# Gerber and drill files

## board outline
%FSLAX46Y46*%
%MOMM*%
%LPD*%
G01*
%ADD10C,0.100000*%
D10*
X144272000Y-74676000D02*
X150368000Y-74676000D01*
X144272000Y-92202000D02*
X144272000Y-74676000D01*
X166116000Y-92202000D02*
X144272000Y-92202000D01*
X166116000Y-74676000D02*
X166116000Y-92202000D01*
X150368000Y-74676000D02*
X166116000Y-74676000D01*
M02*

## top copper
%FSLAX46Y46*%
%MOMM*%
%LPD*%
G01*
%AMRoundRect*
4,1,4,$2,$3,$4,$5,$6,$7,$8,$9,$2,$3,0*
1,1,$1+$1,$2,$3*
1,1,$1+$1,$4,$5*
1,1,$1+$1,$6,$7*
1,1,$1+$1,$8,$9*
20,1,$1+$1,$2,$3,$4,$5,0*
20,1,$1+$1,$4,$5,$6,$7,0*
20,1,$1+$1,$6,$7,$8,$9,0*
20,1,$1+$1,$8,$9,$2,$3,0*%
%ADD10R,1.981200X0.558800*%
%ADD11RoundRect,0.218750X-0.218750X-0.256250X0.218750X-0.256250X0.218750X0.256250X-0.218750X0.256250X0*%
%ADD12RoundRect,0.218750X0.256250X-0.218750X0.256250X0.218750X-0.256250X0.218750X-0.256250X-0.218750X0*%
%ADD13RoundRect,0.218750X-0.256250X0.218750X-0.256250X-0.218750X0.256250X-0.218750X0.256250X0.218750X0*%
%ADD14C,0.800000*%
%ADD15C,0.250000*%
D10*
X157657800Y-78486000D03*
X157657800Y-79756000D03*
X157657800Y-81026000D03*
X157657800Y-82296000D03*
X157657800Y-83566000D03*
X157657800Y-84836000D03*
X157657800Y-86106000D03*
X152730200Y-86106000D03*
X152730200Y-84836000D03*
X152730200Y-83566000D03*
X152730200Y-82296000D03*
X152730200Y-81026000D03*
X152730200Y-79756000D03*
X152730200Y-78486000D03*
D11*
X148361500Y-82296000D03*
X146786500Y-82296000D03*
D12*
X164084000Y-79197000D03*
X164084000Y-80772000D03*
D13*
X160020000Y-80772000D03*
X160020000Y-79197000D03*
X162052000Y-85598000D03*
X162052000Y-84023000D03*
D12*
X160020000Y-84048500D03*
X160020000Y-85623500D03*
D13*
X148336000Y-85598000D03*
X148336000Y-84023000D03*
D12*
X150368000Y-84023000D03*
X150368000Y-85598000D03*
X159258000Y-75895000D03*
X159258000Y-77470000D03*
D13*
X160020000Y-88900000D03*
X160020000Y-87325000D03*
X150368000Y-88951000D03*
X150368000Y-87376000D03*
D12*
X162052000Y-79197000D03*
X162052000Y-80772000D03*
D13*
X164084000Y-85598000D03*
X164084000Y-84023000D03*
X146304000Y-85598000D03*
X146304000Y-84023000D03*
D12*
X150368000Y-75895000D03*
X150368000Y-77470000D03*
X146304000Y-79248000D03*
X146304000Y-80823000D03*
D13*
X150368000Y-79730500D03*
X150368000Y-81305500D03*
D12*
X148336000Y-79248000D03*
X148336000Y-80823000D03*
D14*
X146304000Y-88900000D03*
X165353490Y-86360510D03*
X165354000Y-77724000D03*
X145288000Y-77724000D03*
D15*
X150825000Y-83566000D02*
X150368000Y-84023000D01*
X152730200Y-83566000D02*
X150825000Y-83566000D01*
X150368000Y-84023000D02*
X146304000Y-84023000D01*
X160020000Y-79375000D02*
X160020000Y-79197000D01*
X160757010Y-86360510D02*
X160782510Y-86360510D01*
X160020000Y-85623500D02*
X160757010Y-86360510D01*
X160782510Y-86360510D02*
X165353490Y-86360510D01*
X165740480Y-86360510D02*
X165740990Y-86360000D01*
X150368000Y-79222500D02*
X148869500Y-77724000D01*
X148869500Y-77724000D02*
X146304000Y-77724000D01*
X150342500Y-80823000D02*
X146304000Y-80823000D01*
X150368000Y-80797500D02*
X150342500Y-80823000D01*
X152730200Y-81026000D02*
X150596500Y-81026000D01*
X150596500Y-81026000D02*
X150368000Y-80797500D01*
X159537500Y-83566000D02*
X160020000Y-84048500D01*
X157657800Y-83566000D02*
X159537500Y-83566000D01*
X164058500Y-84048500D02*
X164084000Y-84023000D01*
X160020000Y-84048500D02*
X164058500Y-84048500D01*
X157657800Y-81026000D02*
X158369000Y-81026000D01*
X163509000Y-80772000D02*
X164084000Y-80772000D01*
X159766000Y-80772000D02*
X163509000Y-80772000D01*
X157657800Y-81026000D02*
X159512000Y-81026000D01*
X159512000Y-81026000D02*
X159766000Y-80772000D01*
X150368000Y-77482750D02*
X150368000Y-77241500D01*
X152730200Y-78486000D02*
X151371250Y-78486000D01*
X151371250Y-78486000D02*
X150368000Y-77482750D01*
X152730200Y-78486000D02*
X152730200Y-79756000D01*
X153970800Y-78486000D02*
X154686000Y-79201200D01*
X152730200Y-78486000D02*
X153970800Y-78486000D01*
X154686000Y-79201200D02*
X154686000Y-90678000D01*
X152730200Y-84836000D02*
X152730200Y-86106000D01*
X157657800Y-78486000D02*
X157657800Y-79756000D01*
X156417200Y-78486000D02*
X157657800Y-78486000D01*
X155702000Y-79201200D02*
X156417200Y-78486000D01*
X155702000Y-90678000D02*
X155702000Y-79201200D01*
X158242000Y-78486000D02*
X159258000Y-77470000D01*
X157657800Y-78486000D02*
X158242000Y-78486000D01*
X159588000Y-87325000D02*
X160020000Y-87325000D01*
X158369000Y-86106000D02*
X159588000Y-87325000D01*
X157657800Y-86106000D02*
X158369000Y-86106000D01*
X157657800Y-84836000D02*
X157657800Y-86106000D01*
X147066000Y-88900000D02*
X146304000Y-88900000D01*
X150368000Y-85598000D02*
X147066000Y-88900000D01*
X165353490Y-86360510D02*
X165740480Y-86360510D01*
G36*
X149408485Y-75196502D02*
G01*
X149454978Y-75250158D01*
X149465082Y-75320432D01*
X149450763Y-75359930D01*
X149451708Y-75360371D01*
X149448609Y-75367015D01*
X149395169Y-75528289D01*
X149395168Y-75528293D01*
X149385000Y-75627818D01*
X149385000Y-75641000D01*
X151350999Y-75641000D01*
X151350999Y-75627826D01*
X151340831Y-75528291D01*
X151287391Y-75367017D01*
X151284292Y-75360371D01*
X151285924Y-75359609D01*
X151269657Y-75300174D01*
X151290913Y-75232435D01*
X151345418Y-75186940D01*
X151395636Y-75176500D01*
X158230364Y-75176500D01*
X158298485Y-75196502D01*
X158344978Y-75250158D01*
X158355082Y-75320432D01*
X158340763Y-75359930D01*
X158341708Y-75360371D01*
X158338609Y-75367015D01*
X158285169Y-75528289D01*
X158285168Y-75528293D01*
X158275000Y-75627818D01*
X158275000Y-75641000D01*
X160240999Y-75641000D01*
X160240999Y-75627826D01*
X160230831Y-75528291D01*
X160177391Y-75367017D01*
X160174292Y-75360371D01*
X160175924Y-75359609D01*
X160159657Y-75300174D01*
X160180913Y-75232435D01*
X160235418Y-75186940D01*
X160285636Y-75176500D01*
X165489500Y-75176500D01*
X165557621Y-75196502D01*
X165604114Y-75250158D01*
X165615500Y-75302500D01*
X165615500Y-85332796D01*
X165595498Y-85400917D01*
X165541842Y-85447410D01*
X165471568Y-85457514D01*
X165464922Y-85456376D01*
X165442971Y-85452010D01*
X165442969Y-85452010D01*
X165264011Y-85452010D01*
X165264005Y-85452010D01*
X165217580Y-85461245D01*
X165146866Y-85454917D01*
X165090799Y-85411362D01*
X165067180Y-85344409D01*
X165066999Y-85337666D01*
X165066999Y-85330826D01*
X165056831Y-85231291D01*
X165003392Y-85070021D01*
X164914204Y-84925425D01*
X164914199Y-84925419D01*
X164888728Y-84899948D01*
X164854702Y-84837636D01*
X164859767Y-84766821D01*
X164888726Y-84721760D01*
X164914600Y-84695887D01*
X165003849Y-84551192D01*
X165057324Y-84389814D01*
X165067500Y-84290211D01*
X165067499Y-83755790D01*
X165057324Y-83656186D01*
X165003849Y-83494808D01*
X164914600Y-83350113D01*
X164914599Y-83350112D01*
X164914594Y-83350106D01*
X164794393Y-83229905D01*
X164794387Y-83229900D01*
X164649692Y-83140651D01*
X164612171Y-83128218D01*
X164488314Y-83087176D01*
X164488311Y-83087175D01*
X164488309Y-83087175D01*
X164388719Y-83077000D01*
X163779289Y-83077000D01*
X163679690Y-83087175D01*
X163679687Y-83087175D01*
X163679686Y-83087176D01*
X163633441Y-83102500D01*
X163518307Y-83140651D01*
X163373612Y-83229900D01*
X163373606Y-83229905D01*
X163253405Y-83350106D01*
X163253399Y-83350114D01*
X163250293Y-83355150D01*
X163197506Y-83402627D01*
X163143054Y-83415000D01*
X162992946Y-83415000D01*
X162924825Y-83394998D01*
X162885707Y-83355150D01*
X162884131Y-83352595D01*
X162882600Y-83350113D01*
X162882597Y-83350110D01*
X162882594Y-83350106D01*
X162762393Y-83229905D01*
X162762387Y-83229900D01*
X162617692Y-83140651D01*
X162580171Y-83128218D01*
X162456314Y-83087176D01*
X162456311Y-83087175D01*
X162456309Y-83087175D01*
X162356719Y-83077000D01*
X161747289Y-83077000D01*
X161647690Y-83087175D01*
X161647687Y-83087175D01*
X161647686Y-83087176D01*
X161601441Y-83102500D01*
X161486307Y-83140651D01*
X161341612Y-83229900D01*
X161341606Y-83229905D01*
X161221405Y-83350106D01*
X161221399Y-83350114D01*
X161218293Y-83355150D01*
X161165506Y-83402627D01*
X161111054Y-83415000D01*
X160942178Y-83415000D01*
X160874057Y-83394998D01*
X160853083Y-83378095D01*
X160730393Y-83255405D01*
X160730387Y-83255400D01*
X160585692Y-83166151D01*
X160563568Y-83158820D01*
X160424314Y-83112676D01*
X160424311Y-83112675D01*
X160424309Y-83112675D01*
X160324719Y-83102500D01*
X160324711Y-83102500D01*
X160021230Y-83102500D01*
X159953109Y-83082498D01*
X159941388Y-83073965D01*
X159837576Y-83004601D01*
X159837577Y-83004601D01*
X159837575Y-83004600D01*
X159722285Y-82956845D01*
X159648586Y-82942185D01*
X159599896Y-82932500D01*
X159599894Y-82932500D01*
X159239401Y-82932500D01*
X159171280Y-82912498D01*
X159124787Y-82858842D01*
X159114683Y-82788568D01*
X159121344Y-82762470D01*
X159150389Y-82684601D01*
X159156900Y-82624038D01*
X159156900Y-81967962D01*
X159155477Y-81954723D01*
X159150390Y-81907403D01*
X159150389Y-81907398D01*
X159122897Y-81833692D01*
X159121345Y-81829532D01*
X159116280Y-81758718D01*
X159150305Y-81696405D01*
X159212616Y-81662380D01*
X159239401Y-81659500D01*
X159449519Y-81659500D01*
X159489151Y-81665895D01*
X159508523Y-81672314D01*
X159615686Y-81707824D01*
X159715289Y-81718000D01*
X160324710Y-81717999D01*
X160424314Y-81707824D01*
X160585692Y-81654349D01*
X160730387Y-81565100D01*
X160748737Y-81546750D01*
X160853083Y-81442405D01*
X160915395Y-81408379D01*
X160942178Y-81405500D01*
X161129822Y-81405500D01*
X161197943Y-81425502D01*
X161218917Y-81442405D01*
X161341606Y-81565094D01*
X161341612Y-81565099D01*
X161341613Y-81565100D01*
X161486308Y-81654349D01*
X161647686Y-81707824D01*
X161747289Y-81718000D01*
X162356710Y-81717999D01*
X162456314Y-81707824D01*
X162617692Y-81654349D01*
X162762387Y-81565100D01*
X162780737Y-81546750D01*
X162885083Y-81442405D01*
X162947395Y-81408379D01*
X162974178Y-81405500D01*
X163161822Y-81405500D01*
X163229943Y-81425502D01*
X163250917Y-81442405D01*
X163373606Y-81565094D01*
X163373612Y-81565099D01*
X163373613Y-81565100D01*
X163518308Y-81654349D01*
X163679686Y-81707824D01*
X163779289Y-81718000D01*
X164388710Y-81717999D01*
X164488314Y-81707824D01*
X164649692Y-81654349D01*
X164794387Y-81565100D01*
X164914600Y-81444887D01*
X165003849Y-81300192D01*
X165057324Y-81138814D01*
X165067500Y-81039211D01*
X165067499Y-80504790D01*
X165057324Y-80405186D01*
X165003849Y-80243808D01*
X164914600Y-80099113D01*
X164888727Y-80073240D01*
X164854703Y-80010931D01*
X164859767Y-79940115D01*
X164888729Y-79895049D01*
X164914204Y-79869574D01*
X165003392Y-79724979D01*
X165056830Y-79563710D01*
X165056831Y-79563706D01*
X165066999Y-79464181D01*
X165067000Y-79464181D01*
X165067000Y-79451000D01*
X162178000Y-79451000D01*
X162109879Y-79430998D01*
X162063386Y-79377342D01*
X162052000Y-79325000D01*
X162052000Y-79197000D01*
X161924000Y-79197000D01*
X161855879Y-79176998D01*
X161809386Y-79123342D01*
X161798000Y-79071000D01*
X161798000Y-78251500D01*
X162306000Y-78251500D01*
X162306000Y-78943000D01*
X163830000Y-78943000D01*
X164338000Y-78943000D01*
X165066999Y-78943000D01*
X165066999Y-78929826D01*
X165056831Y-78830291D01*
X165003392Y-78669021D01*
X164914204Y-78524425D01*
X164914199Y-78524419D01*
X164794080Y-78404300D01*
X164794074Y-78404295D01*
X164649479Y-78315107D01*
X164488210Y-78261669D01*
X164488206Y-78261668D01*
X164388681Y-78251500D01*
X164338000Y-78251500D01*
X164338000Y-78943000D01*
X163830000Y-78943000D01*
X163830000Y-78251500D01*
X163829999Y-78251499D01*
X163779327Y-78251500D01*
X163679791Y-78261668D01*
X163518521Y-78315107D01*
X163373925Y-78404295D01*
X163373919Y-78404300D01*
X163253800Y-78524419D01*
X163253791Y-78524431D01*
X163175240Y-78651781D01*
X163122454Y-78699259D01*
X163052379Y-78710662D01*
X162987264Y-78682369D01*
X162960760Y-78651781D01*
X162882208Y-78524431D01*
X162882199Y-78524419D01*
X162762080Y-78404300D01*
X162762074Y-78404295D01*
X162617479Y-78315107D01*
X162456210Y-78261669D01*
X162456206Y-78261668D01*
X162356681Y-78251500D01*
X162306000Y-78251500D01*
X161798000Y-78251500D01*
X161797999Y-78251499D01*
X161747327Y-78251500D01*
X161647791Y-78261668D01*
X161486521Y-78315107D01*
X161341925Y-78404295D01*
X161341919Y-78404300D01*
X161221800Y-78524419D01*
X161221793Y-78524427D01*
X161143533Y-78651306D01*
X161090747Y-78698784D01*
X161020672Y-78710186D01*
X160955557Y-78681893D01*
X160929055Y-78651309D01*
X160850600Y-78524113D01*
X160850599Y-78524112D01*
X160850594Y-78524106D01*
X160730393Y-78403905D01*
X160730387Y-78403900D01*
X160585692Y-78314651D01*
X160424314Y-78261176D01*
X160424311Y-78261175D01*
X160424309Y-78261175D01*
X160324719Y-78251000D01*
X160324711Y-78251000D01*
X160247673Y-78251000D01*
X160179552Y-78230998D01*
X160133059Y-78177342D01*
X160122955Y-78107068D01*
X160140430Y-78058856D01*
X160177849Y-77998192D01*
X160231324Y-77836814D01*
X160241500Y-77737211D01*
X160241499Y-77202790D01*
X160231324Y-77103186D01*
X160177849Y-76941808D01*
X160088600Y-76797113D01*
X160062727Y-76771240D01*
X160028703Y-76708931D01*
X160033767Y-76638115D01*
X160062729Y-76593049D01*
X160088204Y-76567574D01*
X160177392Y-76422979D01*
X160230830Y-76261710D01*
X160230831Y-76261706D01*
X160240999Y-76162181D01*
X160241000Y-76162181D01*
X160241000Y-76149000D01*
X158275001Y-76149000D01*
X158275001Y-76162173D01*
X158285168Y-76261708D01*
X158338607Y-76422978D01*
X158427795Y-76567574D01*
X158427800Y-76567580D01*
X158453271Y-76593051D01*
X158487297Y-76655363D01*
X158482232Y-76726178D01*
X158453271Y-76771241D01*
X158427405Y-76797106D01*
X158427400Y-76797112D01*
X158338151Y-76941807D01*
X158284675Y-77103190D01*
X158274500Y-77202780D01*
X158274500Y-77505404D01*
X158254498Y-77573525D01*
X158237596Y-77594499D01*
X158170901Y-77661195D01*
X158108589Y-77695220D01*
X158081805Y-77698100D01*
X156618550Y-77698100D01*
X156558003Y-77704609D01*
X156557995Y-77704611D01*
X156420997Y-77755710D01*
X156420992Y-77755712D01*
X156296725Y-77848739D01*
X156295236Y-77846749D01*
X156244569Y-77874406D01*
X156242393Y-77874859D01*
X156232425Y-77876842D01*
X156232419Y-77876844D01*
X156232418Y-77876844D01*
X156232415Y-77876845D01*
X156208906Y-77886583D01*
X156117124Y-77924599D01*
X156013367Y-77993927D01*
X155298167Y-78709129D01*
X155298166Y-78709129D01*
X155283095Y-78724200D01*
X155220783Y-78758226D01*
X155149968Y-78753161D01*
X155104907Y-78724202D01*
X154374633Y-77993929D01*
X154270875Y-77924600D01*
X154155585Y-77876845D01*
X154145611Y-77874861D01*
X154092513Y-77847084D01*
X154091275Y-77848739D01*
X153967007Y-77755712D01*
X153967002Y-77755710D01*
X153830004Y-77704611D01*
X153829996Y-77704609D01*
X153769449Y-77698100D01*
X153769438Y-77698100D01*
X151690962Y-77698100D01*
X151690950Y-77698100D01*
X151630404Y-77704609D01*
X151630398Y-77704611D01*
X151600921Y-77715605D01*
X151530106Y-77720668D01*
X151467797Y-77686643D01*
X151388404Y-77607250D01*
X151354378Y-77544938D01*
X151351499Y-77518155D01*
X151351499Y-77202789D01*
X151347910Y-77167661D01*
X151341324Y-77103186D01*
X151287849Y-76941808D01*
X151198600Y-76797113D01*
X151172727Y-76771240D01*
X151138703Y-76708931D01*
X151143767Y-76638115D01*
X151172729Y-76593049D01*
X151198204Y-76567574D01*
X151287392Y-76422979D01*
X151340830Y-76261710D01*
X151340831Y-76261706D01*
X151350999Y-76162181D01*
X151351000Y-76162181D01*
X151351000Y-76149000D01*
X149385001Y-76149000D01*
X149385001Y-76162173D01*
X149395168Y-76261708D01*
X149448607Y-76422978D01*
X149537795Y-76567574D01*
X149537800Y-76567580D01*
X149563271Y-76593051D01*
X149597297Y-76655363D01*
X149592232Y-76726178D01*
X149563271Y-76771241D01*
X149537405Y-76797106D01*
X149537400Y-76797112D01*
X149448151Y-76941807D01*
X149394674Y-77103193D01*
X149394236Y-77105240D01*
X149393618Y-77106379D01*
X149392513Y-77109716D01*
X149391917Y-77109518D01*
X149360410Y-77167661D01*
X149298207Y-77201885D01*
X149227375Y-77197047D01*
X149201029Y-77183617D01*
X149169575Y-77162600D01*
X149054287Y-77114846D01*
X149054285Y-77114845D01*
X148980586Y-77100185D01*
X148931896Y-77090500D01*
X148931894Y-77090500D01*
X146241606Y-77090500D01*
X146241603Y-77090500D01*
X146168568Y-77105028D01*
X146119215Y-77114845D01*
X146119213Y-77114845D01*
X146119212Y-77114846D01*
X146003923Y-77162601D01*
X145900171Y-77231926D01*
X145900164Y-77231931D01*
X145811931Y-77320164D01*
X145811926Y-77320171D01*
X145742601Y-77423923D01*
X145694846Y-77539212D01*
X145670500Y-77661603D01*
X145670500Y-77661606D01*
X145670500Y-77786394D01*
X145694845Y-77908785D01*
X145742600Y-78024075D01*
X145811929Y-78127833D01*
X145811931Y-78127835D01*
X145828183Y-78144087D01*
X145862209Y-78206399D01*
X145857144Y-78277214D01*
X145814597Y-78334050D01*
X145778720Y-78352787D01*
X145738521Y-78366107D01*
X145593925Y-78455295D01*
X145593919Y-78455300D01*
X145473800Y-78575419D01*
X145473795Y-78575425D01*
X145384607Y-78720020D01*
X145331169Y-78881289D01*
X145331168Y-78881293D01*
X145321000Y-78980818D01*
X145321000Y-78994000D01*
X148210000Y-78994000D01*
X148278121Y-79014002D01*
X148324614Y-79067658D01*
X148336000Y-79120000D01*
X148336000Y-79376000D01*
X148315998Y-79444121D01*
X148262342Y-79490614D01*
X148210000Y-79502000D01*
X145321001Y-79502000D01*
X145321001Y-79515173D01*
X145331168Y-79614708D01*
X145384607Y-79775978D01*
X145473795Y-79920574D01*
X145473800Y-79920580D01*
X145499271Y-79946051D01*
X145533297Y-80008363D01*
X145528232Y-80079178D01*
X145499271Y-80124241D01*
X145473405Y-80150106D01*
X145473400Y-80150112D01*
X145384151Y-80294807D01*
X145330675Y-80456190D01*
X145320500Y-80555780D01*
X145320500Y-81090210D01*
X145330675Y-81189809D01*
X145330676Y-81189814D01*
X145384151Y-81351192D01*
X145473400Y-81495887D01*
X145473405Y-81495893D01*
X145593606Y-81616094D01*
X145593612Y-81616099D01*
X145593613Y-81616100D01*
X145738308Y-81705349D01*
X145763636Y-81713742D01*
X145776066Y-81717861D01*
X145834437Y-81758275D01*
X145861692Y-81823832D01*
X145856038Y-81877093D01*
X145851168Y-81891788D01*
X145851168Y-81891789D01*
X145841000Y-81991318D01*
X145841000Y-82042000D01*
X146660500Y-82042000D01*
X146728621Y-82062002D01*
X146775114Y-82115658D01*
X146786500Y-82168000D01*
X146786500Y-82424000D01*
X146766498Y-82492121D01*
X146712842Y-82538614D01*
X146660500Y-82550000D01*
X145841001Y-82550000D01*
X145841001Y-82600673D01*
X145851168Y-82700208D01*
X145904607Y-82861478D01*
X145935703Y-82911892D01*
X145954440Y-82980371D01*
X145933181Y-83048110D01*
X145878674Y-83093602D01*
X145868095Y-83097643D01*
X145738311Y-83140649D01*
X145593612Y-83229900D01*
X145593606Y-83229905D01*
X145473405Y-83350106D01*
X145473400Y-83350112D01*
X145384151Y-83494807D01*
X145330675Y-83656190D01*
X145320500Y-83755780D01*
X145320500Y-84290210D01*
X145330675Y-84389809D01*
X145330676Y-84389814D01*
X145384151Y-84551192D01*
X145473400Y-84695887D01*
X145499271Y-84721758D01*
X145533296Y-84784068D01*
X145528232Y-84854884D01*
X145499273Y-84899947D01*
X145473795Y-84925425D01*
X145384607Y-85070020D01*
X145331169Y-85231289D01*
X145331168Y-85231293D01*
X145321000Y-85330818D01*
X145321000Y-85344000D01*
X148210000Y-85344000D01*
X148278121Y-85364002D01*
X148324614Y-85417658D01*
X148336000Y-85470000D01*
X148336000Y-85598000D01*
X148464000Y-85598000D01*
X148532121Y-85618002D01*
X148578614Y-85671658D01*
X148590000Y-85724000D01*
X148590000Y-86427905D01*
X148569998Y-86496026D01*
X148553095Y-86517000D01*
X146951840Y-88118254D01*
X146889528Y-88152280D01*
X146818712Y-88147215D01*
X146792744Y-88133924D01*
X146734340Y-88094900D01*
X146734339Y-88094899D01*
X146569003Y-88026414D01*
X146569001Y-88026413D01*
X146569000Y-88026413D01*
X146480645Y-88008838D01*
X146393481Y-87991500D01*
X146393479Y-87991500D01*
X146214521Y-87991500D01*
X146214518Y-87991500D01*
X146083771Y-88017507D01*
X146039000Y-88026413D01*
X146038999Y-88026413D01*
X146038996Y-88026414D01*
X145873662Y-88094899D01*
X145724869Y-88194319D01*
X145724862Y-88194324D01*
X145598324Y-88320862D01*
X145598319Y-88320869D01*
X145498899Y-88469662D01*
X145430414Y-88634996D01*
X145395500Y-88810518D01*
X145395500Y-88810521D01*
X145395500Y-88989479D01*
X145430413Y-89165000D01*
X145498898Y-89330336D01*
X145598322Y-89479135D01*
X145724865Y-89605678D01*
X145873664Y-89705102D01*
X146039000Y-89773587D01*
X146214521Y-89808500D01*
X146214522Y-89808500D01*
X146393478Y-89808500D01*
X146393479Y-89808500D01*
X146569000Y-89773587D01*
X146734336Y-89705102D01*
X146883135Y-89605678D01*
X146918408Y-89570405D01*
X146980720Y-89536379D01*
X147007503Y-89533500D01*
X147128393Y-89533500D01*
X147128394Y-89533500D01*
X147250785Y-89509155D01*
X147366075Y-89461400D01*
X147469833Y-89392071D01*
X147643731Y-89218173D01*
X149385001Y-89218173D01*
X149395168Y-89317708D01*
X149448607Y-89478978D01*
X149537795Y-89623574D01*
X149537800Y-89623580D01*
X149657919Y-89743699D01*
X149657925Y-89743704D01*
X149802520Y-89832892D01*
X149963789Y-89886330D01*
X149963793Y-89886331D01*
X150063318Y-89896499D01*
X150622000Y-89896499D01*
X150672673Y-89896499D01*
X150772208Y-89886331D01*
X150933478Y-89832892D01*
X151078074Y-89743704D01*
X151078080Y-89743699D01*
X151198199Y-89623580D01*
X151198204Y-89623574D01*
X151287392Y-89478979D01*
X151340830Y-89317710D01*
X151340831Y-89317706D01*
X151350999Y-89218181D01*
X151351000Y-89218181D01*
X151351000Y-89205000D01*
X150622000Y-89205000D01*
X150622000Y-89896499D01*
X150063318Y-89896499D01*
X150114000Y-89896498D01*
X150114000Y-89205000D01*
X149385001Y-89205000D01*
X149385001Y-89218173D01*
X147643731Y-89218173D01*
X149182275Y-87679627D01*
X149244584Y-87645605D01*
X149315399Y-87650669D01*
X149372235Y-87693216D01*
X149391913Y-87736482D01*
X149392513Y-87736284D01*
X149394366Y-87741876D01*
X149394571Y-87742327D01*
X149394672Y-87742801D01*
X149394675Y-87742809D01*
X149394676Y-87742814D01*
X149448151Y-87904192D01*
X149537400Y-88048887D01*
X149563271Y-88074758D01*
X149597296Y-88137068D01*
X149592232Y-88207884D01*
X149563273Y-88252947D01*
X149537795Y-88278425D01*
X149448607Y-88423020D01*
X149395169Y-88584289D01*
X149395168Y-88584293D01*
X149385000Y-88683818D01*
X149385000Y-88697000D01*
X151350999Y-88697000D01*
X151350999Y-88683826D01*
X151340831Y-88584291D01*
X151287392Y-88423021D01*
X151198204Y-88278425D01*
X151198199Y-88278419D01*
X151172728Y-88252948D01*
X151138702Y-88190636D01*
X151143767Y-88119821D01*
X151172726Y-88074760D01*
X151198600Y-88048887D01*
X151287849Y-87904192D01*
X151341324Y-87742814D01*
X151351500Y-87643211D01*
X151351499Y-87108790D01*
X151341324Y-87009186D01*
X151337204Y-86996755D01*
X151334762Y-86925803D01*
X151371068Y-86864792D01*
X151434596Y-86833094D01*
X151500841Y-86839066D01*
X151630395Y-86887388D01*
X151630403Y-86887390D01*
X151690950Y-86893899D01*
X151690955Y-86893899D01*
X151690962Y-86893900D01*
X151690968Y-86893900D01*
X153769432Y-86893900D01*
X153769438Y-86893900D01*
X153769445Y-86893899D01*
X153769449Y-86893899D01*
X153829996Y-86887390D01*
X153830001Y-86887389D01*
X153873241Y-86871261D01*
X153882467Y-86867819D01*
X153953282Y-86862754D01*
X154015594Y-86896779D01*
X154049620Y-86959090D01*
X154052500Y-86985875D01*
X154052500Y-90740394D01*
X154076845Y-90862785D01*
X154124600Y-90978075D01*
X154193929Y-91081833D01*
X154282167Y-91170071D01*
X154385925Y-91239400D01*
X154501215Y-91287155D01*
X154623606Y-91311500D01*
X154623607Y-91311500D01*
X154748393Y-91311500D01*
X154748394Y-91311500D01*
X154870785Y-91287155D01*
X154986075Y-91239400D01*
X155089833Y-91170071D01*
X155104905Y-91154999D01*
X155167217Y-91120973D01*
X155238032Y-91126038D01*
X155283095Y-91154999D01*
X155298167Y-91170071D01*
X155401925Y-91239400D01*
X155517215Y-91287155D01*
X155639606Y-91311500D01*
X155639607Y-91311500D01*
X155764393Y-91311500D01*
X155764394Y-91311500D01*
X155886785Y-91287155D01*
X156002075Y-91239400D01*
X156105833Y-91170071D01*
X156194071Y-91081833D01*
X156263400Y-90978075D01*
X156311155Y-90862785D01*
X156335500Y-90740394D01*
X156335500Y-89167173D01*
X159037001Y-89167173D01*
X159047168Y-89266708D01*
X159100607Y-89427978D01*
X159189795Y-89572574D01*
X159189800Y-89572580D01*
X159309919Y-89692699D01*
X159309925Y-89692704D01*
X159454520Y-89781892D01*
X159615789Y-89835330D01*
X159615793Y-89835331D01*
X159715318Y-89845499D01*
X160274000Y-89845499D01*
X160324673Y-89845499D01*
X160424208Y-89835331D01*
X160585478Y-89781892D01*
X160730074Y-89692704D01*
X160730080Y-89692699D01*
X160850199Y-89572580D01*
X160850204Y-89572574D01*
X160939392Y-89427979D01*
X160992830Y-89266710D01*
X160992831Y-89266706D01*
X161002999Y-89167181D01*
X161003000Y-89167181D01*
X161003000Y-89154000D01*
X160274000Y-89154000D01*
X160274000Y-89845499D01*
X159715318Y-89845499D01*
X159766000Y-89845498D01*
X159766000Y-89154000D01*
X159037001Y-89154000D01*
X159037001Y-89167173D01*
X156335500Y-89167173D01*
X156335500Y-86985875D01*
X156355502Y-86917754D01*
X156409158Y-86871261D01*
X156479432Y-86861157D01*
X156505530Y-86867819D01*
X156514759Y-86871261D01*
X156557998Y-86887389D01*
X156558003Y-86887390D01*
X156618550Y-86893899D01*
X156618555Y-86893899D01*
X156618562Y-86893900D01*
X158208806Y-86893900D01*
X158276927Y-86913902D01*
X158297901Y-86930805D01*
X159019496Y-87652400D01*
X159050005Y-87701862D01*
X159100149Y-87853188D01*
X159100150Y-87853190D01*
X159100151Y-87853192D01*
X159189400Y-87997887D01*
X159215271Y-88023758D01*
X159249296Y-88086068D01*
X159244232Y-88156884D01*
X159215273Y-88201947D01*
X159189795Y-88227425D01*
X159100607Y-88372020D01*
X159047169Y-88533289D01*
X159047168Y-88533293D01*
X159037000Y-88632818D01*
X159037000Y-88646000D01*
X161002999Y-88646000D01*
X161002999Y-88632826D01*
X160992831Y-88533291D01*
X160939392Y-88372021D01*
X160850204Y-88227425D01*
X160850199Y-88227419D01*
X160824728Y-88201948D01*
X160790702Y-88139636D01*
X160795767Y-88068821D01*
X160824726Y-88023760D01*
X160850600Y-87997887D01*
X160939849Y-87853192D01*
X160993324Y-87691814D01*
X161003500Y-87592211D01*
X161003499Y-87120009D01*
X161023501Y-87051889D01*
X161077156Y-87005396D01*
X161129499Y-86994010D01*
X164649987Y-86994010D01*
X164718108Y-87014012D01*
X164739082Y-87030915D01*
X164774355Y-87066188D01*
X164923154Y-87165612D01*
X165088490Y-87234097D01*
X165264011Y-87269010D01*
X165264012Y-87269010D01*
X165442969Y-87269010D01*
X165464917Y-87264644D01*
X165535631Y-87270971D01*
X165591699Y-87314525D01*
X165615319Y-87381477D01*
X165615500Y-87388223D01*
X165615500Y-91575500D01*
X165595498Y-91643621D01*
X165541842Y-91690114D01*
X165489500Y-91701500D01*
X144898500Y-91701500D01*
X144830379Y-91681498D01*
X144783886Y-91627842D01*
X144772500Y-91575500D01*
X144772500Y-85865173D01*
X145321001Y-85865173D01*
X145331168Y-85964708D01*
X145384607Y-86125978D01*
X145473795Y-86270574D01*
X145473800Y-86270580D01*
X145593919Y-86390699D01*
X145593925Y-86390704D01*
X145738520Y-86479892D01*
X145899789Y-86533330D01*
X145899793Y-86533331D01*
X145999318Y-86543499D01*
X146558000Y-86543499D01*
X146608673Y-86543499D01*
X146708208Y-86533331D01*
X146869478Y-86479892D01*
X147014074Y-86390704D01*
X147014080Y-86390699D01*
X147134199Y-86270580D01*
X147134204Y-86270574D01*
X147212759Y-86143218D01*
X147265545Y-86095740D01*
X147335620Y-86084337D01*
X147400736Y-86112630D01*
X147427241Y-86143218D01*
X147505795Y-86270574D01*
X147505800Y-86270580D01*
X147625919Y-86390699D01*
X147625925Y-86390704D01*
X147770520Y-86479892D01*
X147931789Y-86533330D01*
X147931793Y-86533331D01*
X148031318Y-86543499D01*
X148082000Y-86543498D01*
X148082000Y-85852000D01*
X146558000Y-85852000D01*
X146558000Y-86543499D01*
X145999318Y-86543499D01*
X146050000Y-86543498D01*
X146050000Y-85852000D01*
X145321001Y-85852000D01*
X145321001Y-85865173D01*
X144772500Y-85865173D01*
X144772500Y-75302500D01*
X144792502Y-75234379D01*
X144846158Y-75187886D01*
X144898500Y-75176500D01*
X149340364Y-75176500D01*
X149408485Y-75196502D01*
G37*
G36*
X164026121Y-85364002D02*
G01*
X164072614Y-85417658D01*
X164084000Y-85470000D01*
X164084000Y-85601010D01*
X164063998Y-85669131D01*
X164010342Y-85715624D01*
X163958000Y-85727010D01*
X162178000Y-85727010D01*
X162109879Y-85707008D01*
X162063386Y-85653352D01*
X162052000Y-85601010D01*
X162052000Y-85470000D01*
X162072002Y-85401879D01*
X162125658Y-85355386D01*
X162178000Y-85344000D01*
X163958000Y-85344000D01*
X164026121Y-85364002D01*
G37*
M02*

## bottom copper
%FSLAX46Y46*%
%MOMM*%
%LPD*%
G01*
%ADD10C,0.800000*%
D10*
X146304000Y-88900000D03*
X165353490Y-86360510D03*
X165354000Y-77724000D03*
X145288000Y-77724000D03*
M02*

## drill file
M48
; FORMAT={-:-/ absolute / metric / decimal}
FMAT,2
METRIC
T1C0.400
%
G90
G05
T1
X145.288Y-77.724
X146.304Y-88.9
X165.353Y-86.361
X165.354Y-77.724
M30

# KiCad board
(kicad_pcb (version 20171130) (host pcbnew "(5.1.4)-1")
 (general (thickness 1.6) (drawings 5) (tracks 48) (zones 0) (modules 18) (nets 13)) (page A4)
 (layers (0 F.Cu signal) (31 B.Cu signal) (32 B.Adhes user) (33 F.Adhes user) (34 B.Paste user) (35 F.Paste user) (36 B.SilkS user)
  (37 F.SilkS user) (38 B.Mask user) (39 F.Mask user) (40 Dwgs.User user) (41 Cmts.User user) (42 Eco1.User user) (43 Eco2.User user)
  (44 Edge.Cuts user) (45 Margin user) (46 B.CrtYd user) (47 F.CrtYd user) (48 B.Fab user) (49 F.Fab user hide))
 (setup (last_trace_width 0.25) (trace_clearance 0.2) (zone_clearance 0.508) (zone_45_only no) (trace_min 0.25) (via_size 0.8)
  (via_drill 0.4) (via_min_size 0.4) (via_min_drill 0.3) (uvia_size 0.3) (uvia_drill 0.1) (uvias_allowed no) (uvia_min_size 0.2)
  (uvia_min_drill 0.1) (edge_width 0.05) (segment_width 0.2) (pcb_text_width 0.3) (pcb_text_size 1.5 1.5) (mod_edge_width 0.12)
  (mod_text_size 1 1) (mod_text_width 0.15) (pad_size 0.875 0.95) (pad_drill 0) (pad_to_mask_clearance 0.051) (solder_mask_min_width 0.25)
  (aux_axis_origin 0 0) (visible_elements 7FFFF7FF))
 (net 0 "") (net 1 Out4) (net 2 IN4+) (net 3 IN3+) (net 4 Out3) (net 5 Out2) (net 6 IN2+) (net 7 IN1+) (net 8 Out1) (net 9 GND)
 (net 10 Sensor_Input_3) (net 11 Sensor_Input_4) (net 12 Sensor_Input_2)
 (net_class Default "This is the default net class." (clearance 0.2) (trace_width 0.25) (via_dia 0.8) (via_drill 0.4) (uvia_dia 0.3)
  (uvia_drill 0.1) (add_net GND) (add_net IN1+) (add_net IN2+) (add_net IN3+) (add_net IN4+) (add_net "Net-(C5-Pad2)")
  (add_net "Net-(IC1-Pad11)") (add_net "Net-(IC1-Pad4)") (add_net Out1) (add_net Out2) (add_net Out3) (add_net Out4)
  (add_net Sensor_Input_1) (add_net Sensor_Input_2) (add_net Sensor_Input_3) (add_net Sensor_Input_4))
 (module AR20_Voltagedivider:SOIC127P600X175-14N (layer F.Cu) (at 155.194 82.296)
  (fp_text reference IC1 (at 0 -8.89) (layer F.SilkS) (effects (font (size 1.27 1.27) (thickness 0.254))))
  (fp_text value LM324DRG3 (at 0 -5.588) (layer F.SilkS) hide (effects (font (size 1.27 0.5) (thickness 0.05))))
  (pad 14 smd rect (at 2.4638 -3.81 90) (size 0.5588 1.9812) (layers F.Cu F.Paste F.Mask) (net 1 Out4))
  (pad 13 smd rect (at 2.4638 -2.54 90) (size 0.5588 1.9812) (layers F.Cu F.Paste F.Mask) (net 1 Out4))
  (pad 12 smd rect (at 2.4638 -1.27 90) (size 0.5588 1.9812) (layers F.Cu F.Paste F.Mask) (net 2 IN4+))
  (pad 11 smd rect (at 2.4638 0 90) (size 0.5588 1.9812) (layers F.Cu F.Paste F.Mask))
  (pad 10 smd rect (at 2.4638 1.27 90) (size 0.5588 1.9812) (layers F.Cu F.Paste F.Mask) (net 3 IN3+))
  (pad 9 smd rect (at 2.4638 2.54 90) (size 0.5588 1.9812) (layers F.Cu F.Paste F.Mask) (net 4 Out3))
  (pad 8 smd rect (at 2.4638 3.81 90) (size 0.5588 1.9812) (layers F.Cu F.Paste F.Mask) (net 4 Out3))
  (pad 7 smd rect (at -2.4638 3.81 90) (size 0.5588 1.9812) (layers F.Cu F.Paste F.Mask) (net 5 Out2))
  (pad 6 smd rect (at -2.4638 2.54 90) (size 0.5588 1.9812) (layers F.Cu F.Paste F.Mask) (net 5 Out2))
  (pad 5 smd rect (at -2.4638 1.27 90) (size 0.5588 1.9812) (layers F.Cu F.Paste F.Mask) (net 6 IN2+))
  (pad 4 smd rect (at -2.4638 0 90) (size 0.5588 1.9812) (layers F.Cu F.Paste F.Mask))
  (pad 3 smd rect (at -2.4638 -1.27 90) (size 0.5588 1.9812) (layers F.Cu F.Paste F.Mask) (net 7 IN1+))
  (pad 2 smd rect (at -2.4638 -2.54 90) (size 0.5588 1.9812) (layers F.Cu F.Paste F.Mask) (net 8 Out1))
  (pad 1 smd rect (at -2.4638 -3.81 90) (size 0.5588 1.9812) (layers F.Cu F.Paste F.Mask) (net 8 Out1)))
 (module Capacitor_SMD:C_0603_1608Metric (layer F.Cu) (at 147.574 82.296)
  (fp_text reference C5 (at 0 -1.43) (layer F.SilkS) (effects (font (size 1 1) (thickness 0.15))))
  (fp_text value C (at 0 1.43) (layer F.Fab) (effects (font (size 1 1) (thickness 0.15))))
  (pad 2 smd roundrect (at 0.7875 0) (size 0.875 0.95) (layers F.Cu F.Paste F.Mask) (roundrect_rratio 0.25))
  (pad 1 smd roundrect (at -0.7875 0) (size 0.875 0.95) (layers F.Cu F.Paste F.Mask) (roundrect_rratio 0.25) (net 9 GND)))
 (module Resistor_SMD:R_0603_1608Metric (layer F.Cu) (at 164.084 79.9845 90)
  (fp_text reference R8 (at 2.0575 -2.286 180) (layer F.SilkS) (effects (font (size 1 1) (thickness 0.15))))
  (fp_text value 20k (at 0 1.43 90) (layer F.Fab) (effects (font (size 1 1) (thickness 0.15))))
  (pad 2 smd roundrect (at 0.7875 0 90) (size 0.875 0.95) (layers F.Cu F.Paste F.Mask) (roundrect_rratio 0.25) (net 9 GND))
  (pad 1 smd roundrect (at -0.7875 0 90) (size 0.875 0.95) (layers F.Cu F.Paste F.Mask) (roundrect_rratio 0.25) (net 2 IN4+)))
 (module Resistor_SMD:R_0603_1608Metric (layer F.Cu) (at 160.02 79.9845 270)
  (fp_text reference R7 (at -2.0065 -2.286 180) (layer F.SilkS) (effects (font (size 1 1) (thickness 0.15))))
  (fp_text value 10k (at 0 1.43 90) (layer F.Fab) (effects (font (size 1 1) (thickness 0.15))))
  (pad 2 smd roundrect (at 0.7875 0 270) (size 0.875 0.95) (layers F.Cu F.Paste F.Mask) (roundrect_rratio 0.25) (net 2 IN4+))
  (pad 1 smd roundrect (at -0.7875 0 270) (size 0.875 0.95) (layers F.Cu F.Paste F.Mask) (roundrect_rratio 0.25)))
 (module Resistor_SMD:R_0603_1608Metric (layer F.Cu) (at 162.052 84.8105 270)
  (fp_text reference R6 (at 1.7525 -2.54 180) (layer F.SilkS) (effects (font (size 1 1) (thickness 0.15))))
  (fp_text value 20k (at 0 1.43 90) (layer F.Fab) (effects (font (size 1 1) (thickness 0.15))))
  (pad 2 smd roundrect (at 0.7875 0 270) (size 0.875 0.95) (layers F.Cu F.Paste F.Mask) (roundrect_rratio 0.25) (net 9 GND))
  (pad 1 smd roundrect (at -0.7875 0 270) (size 0.875 0.95) (layers F.Cu F.Paste F.Mask) (roundrect_rratio 0.25) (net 3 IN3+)))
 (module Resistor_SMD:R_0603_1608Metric (layer F.Cu) (at 160.02 84.836 90)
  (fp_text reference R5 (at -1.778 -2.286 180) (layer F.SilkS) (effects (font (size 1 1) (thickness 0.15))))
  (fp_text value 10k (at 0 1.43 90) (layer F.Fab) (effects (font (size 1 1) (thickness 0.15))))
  (pad 2 smd roundrect (at 0.7875 0 90) (size 0.875 0.95) (layers F.Cu F.Paste F.Mask) (roundrect_rratio 0.25) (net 3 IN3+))
  (pad 1 smd roundrect (at -0.7875 0 90) (size 0.875 0.95) (layers F.Cu F.Paste F.Mask) (roundrect_rratio 0.25)))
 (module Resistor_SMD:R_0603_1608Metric (layer F.Cu) (at 148.336 84.8105 270)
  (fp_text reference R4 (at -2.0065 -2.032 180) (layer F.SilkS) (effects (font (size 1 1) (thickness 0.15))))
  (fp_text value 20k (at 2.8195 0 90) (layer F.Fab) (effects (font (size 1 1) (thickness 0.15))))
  (pad 2 smd roundrect (at 0.7875 0 270) (size 0.875 0.95) (layers F.Cu F.Paste F.Mask) (roundrect_rratio 0.25) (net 9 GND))
  (pad 1 smd roundrect (at -0.7875 0 270) (size 0.875 0.95) (layers F.Cu F.Paste F.Mask) (roundrect_rratio 0.25) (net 6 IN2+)))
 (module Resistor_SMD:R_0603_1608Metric (layer F.Cu) (at 150.368 84.8105 90)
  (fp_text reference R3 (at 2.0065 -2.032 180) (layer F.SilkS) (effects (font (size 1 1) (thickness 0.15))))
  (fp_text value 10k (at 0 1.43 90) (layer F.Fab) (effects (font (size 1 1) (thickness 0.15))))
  (pad 2 smd roundrect (at 0.7875 0 90) (size 0.875 0.95) (layers F.Cu F.Paste F.Mask) (roundrect_rratio 0.25) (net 6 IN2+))
  (pad 1 smd roundrect (at -0.7875 0 90) (size 0.875 0.95) (layers F.Cu F.Paste F.Mask) (roundrect_rratio 0.25)))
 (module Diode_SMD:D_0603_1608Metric (layer F.Cu) (at 159.258 76.6825 90)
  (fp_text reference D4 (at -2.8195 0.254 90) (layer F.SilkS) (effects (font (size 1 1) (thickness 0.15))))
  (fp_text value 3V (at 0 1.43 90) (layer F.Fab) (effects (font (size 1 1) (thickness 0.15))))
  (pad 2 smd roundrect (at 0.7875 0 90) (size 0.875 0.95) (layers F.Cu F.Paste F.Mask) (roundrect_rratio 0.25) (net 9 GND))
  (pad 1 smd roundrect (at -0.7875 0 90) (size 0.875 0.95) (layers F.Cu F.Paste F.Mask) (roundrect_rratio 0.25) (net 1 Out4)))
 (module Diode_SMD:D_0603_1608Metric (layer F.Cu) (at 160.02 88.1125 270)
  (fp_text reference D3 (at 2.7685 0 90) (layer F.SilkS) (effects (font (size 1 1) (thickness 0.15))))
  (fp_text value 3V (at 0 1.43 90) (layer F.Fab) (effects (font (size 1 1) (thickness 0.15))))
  (pad 2 smd roundrect (at 0.7875 0 270) (size 0.875 0.95) (layers F.Cu F.Paste F.Mask) (roundrect_rratio 0.25) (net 9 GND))
  (pad 1 smd roundrect (at -0.7875 0 270) (size 0.875 0.95) (layers F.Cu F.Paste F.Mask) (roundrect_rratio 0.25) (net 4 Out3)))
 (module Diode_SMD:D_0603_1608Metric (layer F.Cu) (at 150.368 88.1635 270)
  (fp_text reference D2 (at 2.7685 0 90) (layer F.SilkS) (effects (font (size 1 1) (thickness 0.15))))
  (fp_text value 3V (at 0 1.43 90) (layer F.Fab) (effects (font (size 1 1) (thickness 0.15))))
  (pad 2 smd roundrect (at 0.7875 0 270) (size 0.875 0.95) (layers F.Cu F.Paste F.Mask) (roundrect_rratio 0.25) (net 9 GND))
  (pad 1 smd roundrect (at -0.7875 0 270) (size 0.875 0.95) (layers F.Cu F.Paste F.Mask) (roundrect_rratio 0.25) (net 5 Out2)))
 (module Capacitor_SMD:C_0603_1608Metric (layer F.Cu) (at 162.052 79.9845 90)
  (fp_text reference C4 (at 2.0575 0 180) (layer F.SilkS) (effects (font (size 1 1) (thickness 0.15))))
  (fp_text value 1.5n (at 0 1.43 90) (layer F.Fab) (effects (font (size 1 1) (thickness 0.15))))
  (pad 2 smd roundrect (at 0.7875 0 90) (size 0.875 0.95) (layers F.Cu F.Paste F.Mask) (roundrect_rratio 0.25) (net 9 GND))
  (pad 1 smd roundrect (at -0.7875 0 90) (size 0.875 0.95) (layers F.Cu F.Paste F.Mask) (roundrect_rratio 0.25) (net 2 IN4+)))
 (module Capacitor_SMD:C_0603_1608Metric (layer F.Cu) (at 164.084 84.8105 270)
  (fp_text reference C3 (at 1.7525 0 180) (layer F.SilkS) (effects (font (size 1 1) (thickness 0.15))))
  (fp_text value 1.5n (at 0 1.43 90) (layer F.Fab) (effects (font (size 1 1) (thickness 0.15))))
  (pad 2 smd roundrect (at 0.7875 0 270) (size 0.875 0.95) (layers F.Cu F.Paste F.Mask) (roundrect_rratio 0.25) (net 9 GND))
  (pad 1 smd roundrect (at -0.7875 0 270) (size 0.875 0.95) (layers F.Cu F.Paste F.Mask) (roundrect_rratio 0.25) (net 3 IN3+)))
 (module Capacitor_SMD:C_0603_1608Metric (layer F.Cu) (at 146.304 84.8105 270)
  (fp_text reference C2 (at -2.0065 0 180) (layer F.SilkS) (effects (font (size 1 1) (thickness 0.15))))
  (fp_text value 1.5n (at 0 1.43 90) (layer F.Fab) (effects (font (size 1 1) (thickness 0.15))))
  (pad 2 smd roundrect (at 0.7875 0 270) (size 0.875 0.95) (layers F.Cu F.Paste F.Mask) (roundrect_rratio 0.25) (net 9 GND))
  (pad 1 smd roundrect (at -0.7875 0 270) (size 0.875 0.95) (layers F.Cu F.Paste F.Mask) (roundrect_rratio 0.25) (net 6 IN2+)))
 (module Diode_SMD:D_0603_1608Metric (layer F.Cu) (at 150.368 76.6825 90)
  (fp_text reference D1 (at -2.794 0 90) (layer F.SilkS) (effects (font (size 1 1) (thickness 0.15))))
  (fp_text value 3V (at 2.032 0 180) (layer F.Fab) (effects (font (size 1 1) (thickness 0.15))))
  (pad 2 smd roundrect (at 0.7875 0 90) (size 0.875 0.95) (layers F.Cu F.Paste F.Mask) (roundrect_rratio 0.25) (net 9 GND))
  (pad 1 smd roundrect (at -0.7875 0 90) (size 0.875 0.95) (layers F.Cu F.Paste F.Mask) (roundrect_rratio 0.25) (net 8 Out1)))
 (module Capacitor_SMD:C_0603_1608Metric (layer F.Cu) (at 146.304 80.0355 90)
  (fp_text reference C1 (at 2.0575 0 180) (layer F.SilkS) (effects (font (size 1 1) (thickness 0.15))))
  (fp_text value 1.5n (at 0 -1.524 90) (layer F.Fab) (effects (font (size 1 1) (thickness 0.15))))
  (pad 2 smd roundrect (at 0.7875 0 90) (size 0.875 0.95) (layers F.Cu F.Paste F.Mask) (roundrect_rratio 0.25) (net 9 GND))
  (pad 1 smd roundrect (at -0.7875 0 90) (size 0.875 0.95) (layers F.Cu F.Paste F.Mask) (roundrect_rratio 0.25) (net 7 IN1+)))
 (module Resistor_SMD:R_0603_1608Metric (layer F.Cu) (at 150.368 80.518 270)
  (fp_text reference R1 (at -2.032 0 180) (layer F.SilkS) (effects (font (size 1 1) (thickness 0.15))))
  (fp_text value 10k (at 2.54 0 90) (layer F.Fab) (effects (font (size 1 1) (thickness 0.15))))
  (pad 1 smd roundrect (at -0.7875 0 270) (size 0.875 0.95) (layers F.Cu F.Paste F.Mask) (roundrect_rratio 0.25))
  (pad 2 smd roundrect (at 0.7875 0 270) (size 0.875 0.95) (layers F.Cu F.Paste F.Mask) (roundrect_rratio 0.25) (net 7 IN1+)))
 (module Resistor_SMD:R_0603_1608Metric (layer F.Cu) (at 148.336 80.0355 90)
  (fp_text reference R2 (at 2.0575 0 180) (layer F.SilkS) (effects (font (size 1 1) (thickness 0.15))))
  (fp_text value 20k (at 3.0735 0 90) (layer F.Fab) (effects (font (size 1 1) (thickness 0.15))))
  (pad 2 smd roundrect (at 0.7875 0 90) (size 0.875 0.95) (layers F.Cu F.Paste F.Mask) (roundrect_rratio 0.25) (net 9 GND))
  (pad 1 smd roundrect (at -0.7875 0 90) (size 0.875 0.95) (layers F.Cu F.Paste F.Mask) (roundrect_rratio 0.25) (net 7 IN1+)))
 (gr_line (start 144.272 74.676) (end 150.368 74.676) (layer Edge.Cuts) (width 0.1))
 (gr_line (start 144.272 92.202) (end 144.272 74.676) (layer Edge.Cuts) (width 0.1))
 (gr_line (start 166.116 92.202) (end 144.272 92.202) (layer Edge.Cuts) (width 0.1))
 (gr_line (start 166.116 74.676) (end 166.116 92.202) (layer Edge.Cuts) (width 0.1))
 (gr_line (start 150.368 74.676) (end 166.116 74.676) (layer Edge.Cuts) (width 0.1))
 (segment (start 150.825 83.566) (end 150.368 84.023) (width 0.25) (layer F.Cu) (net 6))
 (segment (start 152.7302 83.566) (end 150.825 83.566) (width 0.25) (layer F.Cu) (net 6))
 (segment (start 150.368 84.023) (end 146.304 84.023) (width 0.25) (layer F.Cu) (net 6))
 (segment (start 160.02 79.375) (end 160.02 79.197) (width 0.25) (layer F.Cu) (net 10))
 (segment (start 160.75701 86.36051) (end 160.78251 86.36051) (width 0.25) (layer F.Cu) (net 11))
 (segment (start 160.02 85.6235) (end 160.75701 86.36051) (width 0.25) (layer F.Cu) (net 11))
 (segment (start 160.78251 86.36051) (end 165.35349 86.36051) (width 0.25) (layer F.Cu) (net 11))
 (segment (start 165.74048 86.36051) (end 165.74099 86.36) (width 0.25) (layer F.Cu) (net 11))
 (segment (start 150.368 79.2225) (end 148.8695 77.724) (width 0.25) (layer F.Cu) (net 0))
 (segment (start 148.8695 77.724) (end 146.304 77.724) (width 0.25) (layer F.Cu) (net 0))
 (segment (start 150.3425 80.823) (end 146.304 80.823) (width 0.25) (layer F.Cu) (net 7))
 (segment (start 150.368 80.7975) (end 150.3425 80.823) (width 0.25) (layer F.Cu) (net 7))
 (segment (start 152.7302 81.026) (end 150.5965 81.026) (width 0.25) (layer F.Cu) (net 7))
 (segment (start 150.5965 81.026) (end 150.368 80.7975) (width 0.25) (layer F.Cu) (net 7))
 (segment (start 159.5375 83.566) (end 160.02 84.0485) (width 0.25) (layer F.Cu) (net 3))
 (segment (start 157.6578 83.566) (end 159.5375 83.566) (width 0.25) (layer F.Cu) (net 3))
 (segment (start 164.0585 84.0485) (end 164.084 84.023) (width 0.25) (layer F.Cu) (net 3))
 (segment (start 160.02 84.0485) (end 164.0585 84.0485) (width 0.25) (layer F.Cu) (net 3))
 (segment (start 157.6578 81.026) (end 158.369 81.026) (width 0.25) (layer F.Cu) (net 2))
 (segment (start 163.509 80.772) (end 164.084 80.772) (width 0.25) (layer F.Cu) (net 2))
 (segment (start 159.766 80.772) (end 163.509 80.772) (width 0.25) (layer F.Cu) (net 2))
 (segment (start 157.6578 81.026) (end 159.512 81.026) (width 0.25) (layer F.Cu) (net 2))
 (segment (start 159.512 81.026) (end 159.766 80.772) (width 0.25) (layer F.Cu) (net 2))
 (segment (start 150.368 77.48275) (end 150.368 77.2415) (width 0.25) (layer F.Cu) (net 8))
 (segment (start 152.7302 78.486) (end 151.37125 78.486) (width 0.25) (layer F.Cu) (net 8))
 (segment (start 151.37125 78.486) (end 150.368 77.48275) (width 0.25) (layer F.Cu) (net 8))
 (segment (start 152.7302 78.486) (end 152.7302 79.756) (width 0.25) (layer F.Cu) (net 8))
 (segment (start 153.9708 78.486) (end 154.686 79.2012) (width 0.25) (layer F.Cu) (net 8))
 (segment (start 152.7302 78.486) (end 153.9708 78.486) (width 0.25) (layer F.Cu) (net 8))
 (segment (start 154.686 79.2012) (end 154.686 90.678) (width 0.25) (layer F.Cu) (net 8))
 (segment (start 152.7302 84.836) (end 152.7302 86.106) (width 0.25) (layer F.Cu) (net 5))
 (segment (start 157.6578 78.486) (end 157.6578 79.756) (width 0.25) (layer F.Cu) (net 1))
 (segment (start 156.4172 78.486) (end 157.6578 78.486) (width 0.25) (layer F.Cu) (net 1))
 (segment (start 155.702 79.2012) (end 156.4172 78.486) (width 0.25) (layer F.Cu) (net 1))
 (segment (start 155.702 90.678) (end 155.702 79.2012) (width 0.25) (layer F.Cu) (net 1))
 (segment (start 158.242 78.486) (end 159.258 77.47) (width 0.25) (layer F.Cu) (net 1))
 (segment (start 157.6578 78.486) (end 158.242 78.486) (width 0.25) (layer F.Cu) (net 1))
 (segment (start 159.588 87.325) (end 160.02 87.325) (width 0.25) (layer F.Cu) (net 4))
 (segment (start 158.369 86.106) (end 159.588 87.325) (width 0.25) (layer F.Cu) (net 4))
 (segment (start 157.6578 86.106) (end 158.369 86.106) (width 0.25) (layer F.Cu) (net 4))
 (segment (start 157.6578 84.836) (end 157.6578 86.106) (width 0.25) (layer F.Cu) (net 4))
 (via (at 146.304 88.9) (size 0.8) (drill 0.4) (layers F.Cu B.Cu) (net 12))
 (segment (start 147.066 88.9) (end 146.304 88.9) (width 0.25) (layer F.Cu) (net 12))
 (segment (start 150.368 85.598) (end 147.066 88.9) (width 0.25) (layer F.Cu) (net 12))
 (segment (start 165.35349 86.36051) (end 165.74048 86.36051) (width 0.25) (layer F.Cu) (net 11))
 (via (at 165.35349 86.36051) (size 0.8) (drill 0.4) (layers F.Cu B.Cu) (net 11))
 (via (at 165.354 77.724) (size 0.8) (drill 0.4) (layers F.Cu B.Cu) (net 9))
 (via (at 145.288 77.724) (size 0.8) (drill 0.4) (layers F.Cu B.Cu) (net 9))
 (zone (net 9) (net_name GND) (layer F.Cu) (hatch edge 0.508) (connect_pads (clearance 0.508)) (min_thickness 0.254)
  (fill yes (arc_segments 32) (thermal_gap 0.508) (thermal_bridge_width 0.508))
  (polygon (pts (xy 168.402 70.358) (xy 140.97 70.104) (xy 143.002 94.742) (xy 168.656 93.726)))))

